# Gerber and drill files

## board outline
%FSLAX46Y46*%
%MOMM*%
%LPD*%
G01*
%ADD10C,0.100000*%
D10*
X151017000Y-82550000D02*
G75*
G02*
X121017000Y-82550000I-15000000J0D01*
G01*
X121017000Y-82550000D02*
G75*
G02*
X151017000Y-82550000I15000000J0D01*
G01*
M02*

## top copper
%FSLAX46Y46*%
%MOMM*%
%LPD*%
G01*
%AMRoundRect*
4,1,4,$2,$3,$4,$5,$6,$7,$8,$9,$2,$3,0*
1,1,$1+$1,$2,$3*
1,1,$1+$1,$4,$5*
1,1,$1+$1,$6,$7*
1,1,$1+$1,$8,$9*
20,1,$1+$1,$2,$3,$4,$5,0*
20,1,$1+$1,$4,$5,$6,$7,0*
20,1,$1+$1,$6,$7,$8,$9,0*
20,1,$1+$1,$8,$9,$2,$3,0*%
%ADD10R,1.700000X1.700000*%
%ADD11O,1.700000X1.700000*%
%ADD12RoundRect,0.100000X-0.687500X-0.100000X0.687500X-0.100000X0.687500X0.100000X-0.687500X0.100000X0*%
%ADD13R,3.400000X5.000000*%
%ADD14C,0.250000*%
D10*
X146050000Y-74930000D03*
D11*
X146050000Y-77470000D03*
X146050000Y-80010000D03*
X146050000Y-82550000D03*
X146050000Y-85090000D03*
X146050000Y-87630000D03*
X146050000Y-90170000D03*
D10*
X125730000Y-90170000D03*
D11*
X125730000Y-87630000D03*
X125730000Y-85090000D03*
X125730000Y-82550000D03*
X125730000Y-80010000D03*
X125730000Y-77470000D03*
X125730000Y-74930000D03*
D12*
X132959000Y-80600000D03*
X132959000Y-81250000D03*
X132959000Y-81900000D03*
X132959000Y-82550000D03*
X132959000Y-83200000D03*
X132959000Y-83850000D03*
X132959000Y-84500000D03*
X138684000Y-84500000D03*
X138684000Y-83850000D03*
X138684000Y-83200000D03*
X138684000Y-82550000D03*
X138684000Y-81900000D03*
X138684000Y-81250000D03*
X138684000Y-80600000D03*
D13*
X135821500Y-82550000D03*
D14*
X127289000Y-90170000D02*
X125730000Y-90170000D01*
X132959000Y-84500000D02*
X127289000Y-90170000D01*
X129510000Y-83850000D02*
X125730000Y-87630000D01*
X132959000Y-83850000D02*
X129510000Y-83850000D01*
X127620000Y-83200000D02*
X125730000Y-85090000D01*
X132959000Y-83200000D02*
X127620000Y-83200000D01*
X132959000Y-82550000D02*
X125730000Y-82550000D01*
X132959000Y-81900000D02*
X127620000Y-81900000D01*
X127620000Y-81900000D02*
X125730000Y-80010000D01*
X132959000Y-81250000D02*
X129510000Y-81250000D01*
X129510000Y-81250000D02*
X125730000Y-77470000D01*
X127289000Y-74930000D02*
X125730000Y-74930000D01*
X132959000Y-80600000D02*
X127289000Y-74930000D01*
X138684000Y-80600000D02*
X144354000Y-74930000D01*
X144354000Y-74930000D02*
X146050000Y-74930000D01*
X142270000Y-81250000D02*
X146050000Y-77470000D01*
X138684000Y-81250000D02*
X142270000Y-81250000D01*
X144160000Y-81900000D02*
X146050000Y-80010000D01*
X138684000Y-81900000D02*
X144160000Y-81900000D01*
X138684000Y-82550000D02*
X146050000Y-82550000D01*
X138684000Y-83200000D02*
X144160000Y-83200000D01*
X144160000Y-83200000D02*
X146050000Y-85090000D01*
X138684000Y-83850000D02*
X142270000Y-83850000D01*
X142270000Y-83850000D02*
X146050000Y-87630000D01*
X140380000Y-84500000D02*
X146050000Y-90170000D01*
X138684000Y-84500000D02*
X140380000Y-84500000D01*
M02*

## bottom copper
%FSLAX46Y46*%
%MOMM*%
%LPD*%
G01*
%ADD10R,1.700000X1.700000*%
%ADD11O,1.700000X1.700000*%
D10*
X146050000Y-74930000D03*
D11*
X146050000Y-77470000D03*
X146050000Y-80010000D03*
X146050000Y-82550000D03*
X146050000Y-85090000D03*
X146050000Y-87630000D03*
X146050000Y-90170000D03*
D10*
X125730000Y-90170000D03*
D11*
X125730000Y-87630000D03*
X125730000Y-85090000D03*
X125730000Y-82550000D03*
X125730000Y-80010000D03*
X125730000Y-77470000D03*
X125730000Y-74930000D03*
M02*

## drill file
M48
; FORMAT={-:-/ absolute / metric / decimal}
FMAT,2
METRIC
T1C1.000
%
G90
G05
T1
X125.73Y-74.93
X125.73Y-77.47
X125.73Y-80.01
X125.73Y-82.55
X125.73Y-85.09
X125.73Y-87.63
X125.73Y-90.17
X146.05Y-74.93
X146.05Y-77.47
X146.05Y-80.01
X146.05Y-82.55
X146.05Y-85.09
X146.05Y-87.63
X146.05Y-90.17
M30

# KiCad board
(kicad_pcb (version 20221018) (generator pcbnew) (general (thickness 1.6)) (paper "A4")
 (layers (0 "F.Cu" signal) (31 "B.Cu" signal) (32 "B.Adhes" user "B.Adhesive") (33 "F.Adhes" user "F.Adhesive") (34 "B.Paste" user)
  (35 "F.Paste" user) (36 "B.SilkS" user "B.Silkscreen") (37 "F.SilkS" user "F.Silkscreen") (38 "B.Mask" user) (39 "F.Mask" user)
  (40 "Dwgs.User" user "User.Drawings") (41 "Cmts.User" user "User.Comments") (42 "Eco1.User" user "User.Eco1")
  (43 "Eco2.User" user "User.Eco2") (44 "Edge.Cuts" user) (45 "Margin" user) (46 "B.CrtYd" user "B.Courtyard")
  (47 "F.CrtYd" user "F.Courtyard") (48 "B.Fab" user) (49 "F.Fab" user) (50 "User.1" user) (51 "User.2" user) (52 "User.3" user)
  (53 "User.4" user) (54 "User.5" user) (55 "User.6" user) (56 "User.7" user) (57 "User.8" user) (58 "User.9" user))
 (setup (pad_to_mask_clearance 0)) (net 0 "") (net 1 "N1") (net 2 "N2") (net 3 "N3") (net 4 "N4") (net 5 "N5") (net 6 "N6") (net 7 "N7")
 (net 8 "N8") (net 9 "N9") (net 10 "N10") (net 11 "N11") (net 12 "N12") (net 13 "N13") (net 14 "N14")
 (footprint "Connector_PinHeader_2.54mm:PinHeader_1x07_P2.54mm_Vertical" (layer "F.Cu") (at 146.05 74.93)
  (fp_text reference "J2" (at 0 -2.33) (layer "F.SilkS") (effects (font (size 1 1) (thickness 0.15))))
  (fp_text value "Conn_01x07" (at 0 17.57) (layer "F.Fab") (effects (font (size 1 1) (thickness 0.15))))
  (pad "1" thru_hole rect (at 0 0) (size 1.7 1.7) (drill 1) (layers "*.Cu" "*.Mask") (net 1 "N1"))
  (pad "2" thru_hole oval (at 0 2.54) (size 1.7 1.7) (drill 1) (layers "*.Cu" "*.Mask") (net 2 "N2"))
  (pad "3" thru_hole oval (at 0 5.08) (size 1.7 1.7) (drill 1) (layers "*.Cu" "*.Mask") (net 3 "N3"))
  (pad "4" thru_hole oval (at 0 7.62) (size 1.7 1.7) (drill 1) (layers "*.Cu" "*.Mask") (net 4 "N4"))
  (pad "5" thru_hole oval (at 0 10.16) (size 1.7 1.7) (drill 1) (layers "*.Cu" "*.Mask") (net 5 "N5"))
  (pad "6" thru_hole oval (at 0 12.7) (size 1.7 1.7) (drill 1) (layers "*.Cu" "*.Mask") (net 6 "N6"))
  (pad "7" thru_hole oval (at 0 15.24) (size 1.7 1.7) (drill 1) (layers "*.Cu" "*.Mask") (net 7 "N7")))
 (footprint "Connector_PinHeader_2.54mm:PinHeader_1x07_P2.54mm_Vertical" (layer "F.Cu") (at 125.73 90.17 180)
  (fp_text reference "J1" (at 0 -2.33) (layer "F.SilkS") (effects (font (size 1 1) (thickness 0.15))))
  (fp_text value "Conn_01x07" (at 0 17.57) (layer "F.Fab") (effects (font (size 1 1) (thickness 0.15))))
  (pad "1" thru_hole rect (at 0 0 180) (size 1.7 1.7) (drill 1) (layers "*.Cu" "*.Mask") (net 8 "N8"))
  (pad "2" thru_hole oval (at 0 2.54 180) (size 1.7 1.7) (drill 1) (layers "*.Cu" "*.Mask") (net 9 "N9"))
  (pad "3" thru_hole oval (at 0 5.08 180) (size 1.7 1.7) (drill 1) (layers "*.Cu" "*.Mask") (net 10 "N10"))
  (pad "4" thru_hole oval (at 0 7.62 180) (size 1.7 1.7) (drill 1) (layers "*.Cu" "*.Mask") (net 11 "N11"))
  (pad "5" thru_hole oval (at 0 10.16 180) (size 1.7 1.7) (drill 1) (layers "*.Cu" "*.Mask") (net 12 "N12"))
  (pad "6" thru_hole oval (at 0 12.7 180) (size 1.7 1.7) (drill 1) (layers "*.Cu" "*.Mask") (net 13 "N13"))
  (pad "7" thru_hole oval (at 0 15.24 180) (size 1.7 1.7) (drill 1) (layers "*.Cu" "*.Mask") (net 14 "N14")))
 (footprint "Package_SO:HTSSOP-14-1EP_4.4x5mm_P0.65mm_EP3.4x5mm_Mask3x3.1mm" (layer "F.Cu") (at 135.8215 82.55)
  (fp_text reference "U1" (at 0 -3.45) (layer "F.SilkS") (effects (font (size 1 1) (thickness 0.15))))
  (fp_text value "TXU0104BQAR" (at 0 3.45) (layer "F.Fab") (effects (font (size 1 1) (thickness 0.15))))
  (pad "" smd roundrect (at -0.75 -0.775) (size 1.21 1.25) (layers "F.Paste") (roundrect_rratio 0.2066123967))
  (pad "" smd roundrect (at -0.75 0.775) (size 1.21 1.25) (layers "F.Paste") (roundrect_rratio 0.2066123967))
  (pad "" smd rect (at 0 0) (size 3 3.1) (layers "F.Mask"))
  (pad "" smd roundrect (at 0.75 -0.775) (size 1.21 1.25) (layers "F.Paste") (roundrect_rratio 0.2066123967))
  (pad "" smd roundrect (at 0.75 0.775) (size 1.21 1.25) (layers "F.Paste") (roundrect_rratio 0.2066123967))
  (pad "1" smd roundrect (at -2.8625 -1.95) (size 1.575 0.4) (layers "F.Cu" "F.Paste" "F.Mask") (roundrect_rratio 0.25) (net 14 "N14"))
  (pad "2" smd roundrect (at -2.8625 -1.3) (size 1.575 0.4) (layers "F.Cu" "F.Paste" "F.Mask") (roundrect_rratio 0.25) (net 13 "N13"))
  (pad "3" smd roundrect (at -2.8625 -0.65) (size 1.575 0.4) (layers "F.Cu" "F.Paste" "F.Mask") (roundrect_rratio 0.25) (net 12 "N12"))
  (pad "4" smd roundrect (at -2.8625 0) (size 1.575 0.4) (layers "F.Cu" "F.Paste" "F.Mask") (roundrect_rratio 0.25) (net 11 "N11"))
  (pad "5" smd roundrect (at -2.8625 0.65) (size 1.575 0.4) (layers "F.Cu" "F.Paste" "F.Mask") (roundrect_rratio 0.25) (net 10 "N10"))
  (pad "6" smd roundrect (at -2.8625 1.3) (size 1.575 0.4) (layers "F.Cu" "F.Paste" "F.Mask") (roundrect_rratio 0.25) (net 9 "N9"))
  (pad "7" smd roundrect (at -2.8625 1.95) (size 1.575 0.4) (layers "F.Cu" "F.Paste" "F.Mask") (roundrect_rratio 0.25) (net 8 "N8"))
  (pad "8" smd roundrect (at 2.8625 1.95) (size 1.575 0.4) (layers "F.Cu" "F.Paste" "F.Mask") (roundrect_rratio 0.25) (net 7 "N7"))
  (pad "9" smd roundrect (at 2.8625 1.3) (size 1.575 0.4) (layers "F.Cu" "F.Paste" "F.Mask") (roundrect_rratio 0.25) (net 6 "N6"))
  (pad "10" smd roundrect (at 2.8625 0.65) (size 1.575 0.4) (layers "F.Cu" "F.Paste" "F.Mask") (roundrect_rratio 0.25) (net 5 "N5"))
  (pad "11" smd roundrect (at 2.8625 0) (size 1.575 0.4) (layers "F.Cu" "F.Paste" "F.Mask") (roundrect_rratio 0.25) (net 4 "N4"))
  (pad "12" smd roundrect (at 2.8625 -0.65) (size 1.575 0.4) (layers "F.Cu" "F.Paste" "F.Mask") (roundrect_rratio 0.25) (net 3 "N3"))
  (pad "13" smd roundrect (at 2.8625 -1.3) (size 1.575 0.4) (layers "F.Cu" "F.Paste" "F.Mask") (roundrect_rratio 0.25) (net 2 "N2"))
  (pad "14" smd roundrect (at 2.8625 -1.95) (size 1.575 0.4) (layers "F.Cu" "F.Paste" "F.Mask") (roundrect_rratio 0.25) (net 1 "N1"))
  (pad "15" smd rect (at 0 0) (size 3.4 5) (layers "F.Cu")))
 (gr_circle (center 136.017 82.55) (end 151.017 82.55) (stroke (width 0.1) (type default)) (fill none) (layer "Edge.Cuts"))
 (segment (start 127.289 90.17) (end 125.73 90.17) (width 0.25) (layer "F.Cu") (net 8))
 (segment (start 132.959 84.5) (end 127.289 90.17) (width 0.25) (layer "F.Cu") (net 8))
 (segment (start 129.51 83.85) (end 125.73 87.63) (width 0.25) (layer "F.Cu") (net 9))
 (segment (start 132.959 83.85) (end 129.51 83.85) (width 0.25) (layer "F.Cu") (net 9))
 (segment (start 127.62 83.2) (end 125.73 85.09) (width 0.25) (layer "F.Cu") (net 10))
 (segment (start 132.959 83.2) (end 127.62 83.2) (width 0.25) (layer "F.Cu") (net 10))
 (segment (start 132.959 82.55) (end 125.73 82.55) (width 0.25) (layer "F.Cu") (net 11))
 (segment (start 132.959 81.9) (end 127.62 81.9) (width 0.25) (layer "F.Cu") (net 12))
 (segment (start 127.62 81.9) (end 125.73 80.01) (width 0.25) (layer "F.Cu") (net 12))
 (segment (start 132.959 81.25) (end 129.51 81.25) (width 0.25) (layer "F.Cu") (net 13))
 (segment (start 129.51 81.25) (end 125.73 77.47) (width 0.25) (layer "F.Cu") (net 13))
 (segment (start 127.289 74.93) (end 125.73 74.93) (width 0.25) (layer "F.Cu") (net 14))
 (segment (start 132.959 80.6) (end 127.289 74.93) (width 0.25) (layer "F.Cu") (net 14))
 (segment (start 138.684 80.6) (end 144.354 74.93) (width 0.25) (layer "F.Cu") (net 1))
 (segment (start 144.354 74.93) (end 146.05 74.93) (width 0.25) (layer "F.Cu") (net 1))
 (segment (start 142.27 81.25) (end 146.05 77.47) (width 0.25) (layer "F.Cu") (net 2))
 (segment (start 138.684 81.25) (end 142.27 81.25) (width 0.25) (layer "F.Cu") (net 2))
 (segment (start 144.16 81.9) (end 146.05 80.01) (width 0.25) (layer "F.Cu") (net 3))
 (segment (start 138.684 81.9) (end 144.16 81.9) (width 0.25) (layer "F.Cu") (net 3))
 (segment (start 138.684 82.55) (end 146.05 82.55) (width 0.25) (layer "F.Cu") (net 4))
 (segment (start 138.684 83.2) (end 144.16 83.2) (width 0.25) (layer "F.Cu") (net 5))
 (segment (start 144.16 83.2) (end 146.05 85.09) (width 0.25) (layer "F.Cu") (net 5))
 (segment (start 138.684 83.85) (end 142.27 83.85) (width 0.25) (layer "F.Cu") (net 6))
 (segment (start 142.27 83.85) (end 146.05 87.63) (width 0.25) (layer "F.Cu") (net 6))
 (segment (start 140.38 84.5) (end 146.05 90.17) (width 0.25) (layer "F.Cu") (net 7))
 (segment (start 138.684 84.5) (end 140.38 84.5) (width 0.25) (layer "F.Cu") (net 7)))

